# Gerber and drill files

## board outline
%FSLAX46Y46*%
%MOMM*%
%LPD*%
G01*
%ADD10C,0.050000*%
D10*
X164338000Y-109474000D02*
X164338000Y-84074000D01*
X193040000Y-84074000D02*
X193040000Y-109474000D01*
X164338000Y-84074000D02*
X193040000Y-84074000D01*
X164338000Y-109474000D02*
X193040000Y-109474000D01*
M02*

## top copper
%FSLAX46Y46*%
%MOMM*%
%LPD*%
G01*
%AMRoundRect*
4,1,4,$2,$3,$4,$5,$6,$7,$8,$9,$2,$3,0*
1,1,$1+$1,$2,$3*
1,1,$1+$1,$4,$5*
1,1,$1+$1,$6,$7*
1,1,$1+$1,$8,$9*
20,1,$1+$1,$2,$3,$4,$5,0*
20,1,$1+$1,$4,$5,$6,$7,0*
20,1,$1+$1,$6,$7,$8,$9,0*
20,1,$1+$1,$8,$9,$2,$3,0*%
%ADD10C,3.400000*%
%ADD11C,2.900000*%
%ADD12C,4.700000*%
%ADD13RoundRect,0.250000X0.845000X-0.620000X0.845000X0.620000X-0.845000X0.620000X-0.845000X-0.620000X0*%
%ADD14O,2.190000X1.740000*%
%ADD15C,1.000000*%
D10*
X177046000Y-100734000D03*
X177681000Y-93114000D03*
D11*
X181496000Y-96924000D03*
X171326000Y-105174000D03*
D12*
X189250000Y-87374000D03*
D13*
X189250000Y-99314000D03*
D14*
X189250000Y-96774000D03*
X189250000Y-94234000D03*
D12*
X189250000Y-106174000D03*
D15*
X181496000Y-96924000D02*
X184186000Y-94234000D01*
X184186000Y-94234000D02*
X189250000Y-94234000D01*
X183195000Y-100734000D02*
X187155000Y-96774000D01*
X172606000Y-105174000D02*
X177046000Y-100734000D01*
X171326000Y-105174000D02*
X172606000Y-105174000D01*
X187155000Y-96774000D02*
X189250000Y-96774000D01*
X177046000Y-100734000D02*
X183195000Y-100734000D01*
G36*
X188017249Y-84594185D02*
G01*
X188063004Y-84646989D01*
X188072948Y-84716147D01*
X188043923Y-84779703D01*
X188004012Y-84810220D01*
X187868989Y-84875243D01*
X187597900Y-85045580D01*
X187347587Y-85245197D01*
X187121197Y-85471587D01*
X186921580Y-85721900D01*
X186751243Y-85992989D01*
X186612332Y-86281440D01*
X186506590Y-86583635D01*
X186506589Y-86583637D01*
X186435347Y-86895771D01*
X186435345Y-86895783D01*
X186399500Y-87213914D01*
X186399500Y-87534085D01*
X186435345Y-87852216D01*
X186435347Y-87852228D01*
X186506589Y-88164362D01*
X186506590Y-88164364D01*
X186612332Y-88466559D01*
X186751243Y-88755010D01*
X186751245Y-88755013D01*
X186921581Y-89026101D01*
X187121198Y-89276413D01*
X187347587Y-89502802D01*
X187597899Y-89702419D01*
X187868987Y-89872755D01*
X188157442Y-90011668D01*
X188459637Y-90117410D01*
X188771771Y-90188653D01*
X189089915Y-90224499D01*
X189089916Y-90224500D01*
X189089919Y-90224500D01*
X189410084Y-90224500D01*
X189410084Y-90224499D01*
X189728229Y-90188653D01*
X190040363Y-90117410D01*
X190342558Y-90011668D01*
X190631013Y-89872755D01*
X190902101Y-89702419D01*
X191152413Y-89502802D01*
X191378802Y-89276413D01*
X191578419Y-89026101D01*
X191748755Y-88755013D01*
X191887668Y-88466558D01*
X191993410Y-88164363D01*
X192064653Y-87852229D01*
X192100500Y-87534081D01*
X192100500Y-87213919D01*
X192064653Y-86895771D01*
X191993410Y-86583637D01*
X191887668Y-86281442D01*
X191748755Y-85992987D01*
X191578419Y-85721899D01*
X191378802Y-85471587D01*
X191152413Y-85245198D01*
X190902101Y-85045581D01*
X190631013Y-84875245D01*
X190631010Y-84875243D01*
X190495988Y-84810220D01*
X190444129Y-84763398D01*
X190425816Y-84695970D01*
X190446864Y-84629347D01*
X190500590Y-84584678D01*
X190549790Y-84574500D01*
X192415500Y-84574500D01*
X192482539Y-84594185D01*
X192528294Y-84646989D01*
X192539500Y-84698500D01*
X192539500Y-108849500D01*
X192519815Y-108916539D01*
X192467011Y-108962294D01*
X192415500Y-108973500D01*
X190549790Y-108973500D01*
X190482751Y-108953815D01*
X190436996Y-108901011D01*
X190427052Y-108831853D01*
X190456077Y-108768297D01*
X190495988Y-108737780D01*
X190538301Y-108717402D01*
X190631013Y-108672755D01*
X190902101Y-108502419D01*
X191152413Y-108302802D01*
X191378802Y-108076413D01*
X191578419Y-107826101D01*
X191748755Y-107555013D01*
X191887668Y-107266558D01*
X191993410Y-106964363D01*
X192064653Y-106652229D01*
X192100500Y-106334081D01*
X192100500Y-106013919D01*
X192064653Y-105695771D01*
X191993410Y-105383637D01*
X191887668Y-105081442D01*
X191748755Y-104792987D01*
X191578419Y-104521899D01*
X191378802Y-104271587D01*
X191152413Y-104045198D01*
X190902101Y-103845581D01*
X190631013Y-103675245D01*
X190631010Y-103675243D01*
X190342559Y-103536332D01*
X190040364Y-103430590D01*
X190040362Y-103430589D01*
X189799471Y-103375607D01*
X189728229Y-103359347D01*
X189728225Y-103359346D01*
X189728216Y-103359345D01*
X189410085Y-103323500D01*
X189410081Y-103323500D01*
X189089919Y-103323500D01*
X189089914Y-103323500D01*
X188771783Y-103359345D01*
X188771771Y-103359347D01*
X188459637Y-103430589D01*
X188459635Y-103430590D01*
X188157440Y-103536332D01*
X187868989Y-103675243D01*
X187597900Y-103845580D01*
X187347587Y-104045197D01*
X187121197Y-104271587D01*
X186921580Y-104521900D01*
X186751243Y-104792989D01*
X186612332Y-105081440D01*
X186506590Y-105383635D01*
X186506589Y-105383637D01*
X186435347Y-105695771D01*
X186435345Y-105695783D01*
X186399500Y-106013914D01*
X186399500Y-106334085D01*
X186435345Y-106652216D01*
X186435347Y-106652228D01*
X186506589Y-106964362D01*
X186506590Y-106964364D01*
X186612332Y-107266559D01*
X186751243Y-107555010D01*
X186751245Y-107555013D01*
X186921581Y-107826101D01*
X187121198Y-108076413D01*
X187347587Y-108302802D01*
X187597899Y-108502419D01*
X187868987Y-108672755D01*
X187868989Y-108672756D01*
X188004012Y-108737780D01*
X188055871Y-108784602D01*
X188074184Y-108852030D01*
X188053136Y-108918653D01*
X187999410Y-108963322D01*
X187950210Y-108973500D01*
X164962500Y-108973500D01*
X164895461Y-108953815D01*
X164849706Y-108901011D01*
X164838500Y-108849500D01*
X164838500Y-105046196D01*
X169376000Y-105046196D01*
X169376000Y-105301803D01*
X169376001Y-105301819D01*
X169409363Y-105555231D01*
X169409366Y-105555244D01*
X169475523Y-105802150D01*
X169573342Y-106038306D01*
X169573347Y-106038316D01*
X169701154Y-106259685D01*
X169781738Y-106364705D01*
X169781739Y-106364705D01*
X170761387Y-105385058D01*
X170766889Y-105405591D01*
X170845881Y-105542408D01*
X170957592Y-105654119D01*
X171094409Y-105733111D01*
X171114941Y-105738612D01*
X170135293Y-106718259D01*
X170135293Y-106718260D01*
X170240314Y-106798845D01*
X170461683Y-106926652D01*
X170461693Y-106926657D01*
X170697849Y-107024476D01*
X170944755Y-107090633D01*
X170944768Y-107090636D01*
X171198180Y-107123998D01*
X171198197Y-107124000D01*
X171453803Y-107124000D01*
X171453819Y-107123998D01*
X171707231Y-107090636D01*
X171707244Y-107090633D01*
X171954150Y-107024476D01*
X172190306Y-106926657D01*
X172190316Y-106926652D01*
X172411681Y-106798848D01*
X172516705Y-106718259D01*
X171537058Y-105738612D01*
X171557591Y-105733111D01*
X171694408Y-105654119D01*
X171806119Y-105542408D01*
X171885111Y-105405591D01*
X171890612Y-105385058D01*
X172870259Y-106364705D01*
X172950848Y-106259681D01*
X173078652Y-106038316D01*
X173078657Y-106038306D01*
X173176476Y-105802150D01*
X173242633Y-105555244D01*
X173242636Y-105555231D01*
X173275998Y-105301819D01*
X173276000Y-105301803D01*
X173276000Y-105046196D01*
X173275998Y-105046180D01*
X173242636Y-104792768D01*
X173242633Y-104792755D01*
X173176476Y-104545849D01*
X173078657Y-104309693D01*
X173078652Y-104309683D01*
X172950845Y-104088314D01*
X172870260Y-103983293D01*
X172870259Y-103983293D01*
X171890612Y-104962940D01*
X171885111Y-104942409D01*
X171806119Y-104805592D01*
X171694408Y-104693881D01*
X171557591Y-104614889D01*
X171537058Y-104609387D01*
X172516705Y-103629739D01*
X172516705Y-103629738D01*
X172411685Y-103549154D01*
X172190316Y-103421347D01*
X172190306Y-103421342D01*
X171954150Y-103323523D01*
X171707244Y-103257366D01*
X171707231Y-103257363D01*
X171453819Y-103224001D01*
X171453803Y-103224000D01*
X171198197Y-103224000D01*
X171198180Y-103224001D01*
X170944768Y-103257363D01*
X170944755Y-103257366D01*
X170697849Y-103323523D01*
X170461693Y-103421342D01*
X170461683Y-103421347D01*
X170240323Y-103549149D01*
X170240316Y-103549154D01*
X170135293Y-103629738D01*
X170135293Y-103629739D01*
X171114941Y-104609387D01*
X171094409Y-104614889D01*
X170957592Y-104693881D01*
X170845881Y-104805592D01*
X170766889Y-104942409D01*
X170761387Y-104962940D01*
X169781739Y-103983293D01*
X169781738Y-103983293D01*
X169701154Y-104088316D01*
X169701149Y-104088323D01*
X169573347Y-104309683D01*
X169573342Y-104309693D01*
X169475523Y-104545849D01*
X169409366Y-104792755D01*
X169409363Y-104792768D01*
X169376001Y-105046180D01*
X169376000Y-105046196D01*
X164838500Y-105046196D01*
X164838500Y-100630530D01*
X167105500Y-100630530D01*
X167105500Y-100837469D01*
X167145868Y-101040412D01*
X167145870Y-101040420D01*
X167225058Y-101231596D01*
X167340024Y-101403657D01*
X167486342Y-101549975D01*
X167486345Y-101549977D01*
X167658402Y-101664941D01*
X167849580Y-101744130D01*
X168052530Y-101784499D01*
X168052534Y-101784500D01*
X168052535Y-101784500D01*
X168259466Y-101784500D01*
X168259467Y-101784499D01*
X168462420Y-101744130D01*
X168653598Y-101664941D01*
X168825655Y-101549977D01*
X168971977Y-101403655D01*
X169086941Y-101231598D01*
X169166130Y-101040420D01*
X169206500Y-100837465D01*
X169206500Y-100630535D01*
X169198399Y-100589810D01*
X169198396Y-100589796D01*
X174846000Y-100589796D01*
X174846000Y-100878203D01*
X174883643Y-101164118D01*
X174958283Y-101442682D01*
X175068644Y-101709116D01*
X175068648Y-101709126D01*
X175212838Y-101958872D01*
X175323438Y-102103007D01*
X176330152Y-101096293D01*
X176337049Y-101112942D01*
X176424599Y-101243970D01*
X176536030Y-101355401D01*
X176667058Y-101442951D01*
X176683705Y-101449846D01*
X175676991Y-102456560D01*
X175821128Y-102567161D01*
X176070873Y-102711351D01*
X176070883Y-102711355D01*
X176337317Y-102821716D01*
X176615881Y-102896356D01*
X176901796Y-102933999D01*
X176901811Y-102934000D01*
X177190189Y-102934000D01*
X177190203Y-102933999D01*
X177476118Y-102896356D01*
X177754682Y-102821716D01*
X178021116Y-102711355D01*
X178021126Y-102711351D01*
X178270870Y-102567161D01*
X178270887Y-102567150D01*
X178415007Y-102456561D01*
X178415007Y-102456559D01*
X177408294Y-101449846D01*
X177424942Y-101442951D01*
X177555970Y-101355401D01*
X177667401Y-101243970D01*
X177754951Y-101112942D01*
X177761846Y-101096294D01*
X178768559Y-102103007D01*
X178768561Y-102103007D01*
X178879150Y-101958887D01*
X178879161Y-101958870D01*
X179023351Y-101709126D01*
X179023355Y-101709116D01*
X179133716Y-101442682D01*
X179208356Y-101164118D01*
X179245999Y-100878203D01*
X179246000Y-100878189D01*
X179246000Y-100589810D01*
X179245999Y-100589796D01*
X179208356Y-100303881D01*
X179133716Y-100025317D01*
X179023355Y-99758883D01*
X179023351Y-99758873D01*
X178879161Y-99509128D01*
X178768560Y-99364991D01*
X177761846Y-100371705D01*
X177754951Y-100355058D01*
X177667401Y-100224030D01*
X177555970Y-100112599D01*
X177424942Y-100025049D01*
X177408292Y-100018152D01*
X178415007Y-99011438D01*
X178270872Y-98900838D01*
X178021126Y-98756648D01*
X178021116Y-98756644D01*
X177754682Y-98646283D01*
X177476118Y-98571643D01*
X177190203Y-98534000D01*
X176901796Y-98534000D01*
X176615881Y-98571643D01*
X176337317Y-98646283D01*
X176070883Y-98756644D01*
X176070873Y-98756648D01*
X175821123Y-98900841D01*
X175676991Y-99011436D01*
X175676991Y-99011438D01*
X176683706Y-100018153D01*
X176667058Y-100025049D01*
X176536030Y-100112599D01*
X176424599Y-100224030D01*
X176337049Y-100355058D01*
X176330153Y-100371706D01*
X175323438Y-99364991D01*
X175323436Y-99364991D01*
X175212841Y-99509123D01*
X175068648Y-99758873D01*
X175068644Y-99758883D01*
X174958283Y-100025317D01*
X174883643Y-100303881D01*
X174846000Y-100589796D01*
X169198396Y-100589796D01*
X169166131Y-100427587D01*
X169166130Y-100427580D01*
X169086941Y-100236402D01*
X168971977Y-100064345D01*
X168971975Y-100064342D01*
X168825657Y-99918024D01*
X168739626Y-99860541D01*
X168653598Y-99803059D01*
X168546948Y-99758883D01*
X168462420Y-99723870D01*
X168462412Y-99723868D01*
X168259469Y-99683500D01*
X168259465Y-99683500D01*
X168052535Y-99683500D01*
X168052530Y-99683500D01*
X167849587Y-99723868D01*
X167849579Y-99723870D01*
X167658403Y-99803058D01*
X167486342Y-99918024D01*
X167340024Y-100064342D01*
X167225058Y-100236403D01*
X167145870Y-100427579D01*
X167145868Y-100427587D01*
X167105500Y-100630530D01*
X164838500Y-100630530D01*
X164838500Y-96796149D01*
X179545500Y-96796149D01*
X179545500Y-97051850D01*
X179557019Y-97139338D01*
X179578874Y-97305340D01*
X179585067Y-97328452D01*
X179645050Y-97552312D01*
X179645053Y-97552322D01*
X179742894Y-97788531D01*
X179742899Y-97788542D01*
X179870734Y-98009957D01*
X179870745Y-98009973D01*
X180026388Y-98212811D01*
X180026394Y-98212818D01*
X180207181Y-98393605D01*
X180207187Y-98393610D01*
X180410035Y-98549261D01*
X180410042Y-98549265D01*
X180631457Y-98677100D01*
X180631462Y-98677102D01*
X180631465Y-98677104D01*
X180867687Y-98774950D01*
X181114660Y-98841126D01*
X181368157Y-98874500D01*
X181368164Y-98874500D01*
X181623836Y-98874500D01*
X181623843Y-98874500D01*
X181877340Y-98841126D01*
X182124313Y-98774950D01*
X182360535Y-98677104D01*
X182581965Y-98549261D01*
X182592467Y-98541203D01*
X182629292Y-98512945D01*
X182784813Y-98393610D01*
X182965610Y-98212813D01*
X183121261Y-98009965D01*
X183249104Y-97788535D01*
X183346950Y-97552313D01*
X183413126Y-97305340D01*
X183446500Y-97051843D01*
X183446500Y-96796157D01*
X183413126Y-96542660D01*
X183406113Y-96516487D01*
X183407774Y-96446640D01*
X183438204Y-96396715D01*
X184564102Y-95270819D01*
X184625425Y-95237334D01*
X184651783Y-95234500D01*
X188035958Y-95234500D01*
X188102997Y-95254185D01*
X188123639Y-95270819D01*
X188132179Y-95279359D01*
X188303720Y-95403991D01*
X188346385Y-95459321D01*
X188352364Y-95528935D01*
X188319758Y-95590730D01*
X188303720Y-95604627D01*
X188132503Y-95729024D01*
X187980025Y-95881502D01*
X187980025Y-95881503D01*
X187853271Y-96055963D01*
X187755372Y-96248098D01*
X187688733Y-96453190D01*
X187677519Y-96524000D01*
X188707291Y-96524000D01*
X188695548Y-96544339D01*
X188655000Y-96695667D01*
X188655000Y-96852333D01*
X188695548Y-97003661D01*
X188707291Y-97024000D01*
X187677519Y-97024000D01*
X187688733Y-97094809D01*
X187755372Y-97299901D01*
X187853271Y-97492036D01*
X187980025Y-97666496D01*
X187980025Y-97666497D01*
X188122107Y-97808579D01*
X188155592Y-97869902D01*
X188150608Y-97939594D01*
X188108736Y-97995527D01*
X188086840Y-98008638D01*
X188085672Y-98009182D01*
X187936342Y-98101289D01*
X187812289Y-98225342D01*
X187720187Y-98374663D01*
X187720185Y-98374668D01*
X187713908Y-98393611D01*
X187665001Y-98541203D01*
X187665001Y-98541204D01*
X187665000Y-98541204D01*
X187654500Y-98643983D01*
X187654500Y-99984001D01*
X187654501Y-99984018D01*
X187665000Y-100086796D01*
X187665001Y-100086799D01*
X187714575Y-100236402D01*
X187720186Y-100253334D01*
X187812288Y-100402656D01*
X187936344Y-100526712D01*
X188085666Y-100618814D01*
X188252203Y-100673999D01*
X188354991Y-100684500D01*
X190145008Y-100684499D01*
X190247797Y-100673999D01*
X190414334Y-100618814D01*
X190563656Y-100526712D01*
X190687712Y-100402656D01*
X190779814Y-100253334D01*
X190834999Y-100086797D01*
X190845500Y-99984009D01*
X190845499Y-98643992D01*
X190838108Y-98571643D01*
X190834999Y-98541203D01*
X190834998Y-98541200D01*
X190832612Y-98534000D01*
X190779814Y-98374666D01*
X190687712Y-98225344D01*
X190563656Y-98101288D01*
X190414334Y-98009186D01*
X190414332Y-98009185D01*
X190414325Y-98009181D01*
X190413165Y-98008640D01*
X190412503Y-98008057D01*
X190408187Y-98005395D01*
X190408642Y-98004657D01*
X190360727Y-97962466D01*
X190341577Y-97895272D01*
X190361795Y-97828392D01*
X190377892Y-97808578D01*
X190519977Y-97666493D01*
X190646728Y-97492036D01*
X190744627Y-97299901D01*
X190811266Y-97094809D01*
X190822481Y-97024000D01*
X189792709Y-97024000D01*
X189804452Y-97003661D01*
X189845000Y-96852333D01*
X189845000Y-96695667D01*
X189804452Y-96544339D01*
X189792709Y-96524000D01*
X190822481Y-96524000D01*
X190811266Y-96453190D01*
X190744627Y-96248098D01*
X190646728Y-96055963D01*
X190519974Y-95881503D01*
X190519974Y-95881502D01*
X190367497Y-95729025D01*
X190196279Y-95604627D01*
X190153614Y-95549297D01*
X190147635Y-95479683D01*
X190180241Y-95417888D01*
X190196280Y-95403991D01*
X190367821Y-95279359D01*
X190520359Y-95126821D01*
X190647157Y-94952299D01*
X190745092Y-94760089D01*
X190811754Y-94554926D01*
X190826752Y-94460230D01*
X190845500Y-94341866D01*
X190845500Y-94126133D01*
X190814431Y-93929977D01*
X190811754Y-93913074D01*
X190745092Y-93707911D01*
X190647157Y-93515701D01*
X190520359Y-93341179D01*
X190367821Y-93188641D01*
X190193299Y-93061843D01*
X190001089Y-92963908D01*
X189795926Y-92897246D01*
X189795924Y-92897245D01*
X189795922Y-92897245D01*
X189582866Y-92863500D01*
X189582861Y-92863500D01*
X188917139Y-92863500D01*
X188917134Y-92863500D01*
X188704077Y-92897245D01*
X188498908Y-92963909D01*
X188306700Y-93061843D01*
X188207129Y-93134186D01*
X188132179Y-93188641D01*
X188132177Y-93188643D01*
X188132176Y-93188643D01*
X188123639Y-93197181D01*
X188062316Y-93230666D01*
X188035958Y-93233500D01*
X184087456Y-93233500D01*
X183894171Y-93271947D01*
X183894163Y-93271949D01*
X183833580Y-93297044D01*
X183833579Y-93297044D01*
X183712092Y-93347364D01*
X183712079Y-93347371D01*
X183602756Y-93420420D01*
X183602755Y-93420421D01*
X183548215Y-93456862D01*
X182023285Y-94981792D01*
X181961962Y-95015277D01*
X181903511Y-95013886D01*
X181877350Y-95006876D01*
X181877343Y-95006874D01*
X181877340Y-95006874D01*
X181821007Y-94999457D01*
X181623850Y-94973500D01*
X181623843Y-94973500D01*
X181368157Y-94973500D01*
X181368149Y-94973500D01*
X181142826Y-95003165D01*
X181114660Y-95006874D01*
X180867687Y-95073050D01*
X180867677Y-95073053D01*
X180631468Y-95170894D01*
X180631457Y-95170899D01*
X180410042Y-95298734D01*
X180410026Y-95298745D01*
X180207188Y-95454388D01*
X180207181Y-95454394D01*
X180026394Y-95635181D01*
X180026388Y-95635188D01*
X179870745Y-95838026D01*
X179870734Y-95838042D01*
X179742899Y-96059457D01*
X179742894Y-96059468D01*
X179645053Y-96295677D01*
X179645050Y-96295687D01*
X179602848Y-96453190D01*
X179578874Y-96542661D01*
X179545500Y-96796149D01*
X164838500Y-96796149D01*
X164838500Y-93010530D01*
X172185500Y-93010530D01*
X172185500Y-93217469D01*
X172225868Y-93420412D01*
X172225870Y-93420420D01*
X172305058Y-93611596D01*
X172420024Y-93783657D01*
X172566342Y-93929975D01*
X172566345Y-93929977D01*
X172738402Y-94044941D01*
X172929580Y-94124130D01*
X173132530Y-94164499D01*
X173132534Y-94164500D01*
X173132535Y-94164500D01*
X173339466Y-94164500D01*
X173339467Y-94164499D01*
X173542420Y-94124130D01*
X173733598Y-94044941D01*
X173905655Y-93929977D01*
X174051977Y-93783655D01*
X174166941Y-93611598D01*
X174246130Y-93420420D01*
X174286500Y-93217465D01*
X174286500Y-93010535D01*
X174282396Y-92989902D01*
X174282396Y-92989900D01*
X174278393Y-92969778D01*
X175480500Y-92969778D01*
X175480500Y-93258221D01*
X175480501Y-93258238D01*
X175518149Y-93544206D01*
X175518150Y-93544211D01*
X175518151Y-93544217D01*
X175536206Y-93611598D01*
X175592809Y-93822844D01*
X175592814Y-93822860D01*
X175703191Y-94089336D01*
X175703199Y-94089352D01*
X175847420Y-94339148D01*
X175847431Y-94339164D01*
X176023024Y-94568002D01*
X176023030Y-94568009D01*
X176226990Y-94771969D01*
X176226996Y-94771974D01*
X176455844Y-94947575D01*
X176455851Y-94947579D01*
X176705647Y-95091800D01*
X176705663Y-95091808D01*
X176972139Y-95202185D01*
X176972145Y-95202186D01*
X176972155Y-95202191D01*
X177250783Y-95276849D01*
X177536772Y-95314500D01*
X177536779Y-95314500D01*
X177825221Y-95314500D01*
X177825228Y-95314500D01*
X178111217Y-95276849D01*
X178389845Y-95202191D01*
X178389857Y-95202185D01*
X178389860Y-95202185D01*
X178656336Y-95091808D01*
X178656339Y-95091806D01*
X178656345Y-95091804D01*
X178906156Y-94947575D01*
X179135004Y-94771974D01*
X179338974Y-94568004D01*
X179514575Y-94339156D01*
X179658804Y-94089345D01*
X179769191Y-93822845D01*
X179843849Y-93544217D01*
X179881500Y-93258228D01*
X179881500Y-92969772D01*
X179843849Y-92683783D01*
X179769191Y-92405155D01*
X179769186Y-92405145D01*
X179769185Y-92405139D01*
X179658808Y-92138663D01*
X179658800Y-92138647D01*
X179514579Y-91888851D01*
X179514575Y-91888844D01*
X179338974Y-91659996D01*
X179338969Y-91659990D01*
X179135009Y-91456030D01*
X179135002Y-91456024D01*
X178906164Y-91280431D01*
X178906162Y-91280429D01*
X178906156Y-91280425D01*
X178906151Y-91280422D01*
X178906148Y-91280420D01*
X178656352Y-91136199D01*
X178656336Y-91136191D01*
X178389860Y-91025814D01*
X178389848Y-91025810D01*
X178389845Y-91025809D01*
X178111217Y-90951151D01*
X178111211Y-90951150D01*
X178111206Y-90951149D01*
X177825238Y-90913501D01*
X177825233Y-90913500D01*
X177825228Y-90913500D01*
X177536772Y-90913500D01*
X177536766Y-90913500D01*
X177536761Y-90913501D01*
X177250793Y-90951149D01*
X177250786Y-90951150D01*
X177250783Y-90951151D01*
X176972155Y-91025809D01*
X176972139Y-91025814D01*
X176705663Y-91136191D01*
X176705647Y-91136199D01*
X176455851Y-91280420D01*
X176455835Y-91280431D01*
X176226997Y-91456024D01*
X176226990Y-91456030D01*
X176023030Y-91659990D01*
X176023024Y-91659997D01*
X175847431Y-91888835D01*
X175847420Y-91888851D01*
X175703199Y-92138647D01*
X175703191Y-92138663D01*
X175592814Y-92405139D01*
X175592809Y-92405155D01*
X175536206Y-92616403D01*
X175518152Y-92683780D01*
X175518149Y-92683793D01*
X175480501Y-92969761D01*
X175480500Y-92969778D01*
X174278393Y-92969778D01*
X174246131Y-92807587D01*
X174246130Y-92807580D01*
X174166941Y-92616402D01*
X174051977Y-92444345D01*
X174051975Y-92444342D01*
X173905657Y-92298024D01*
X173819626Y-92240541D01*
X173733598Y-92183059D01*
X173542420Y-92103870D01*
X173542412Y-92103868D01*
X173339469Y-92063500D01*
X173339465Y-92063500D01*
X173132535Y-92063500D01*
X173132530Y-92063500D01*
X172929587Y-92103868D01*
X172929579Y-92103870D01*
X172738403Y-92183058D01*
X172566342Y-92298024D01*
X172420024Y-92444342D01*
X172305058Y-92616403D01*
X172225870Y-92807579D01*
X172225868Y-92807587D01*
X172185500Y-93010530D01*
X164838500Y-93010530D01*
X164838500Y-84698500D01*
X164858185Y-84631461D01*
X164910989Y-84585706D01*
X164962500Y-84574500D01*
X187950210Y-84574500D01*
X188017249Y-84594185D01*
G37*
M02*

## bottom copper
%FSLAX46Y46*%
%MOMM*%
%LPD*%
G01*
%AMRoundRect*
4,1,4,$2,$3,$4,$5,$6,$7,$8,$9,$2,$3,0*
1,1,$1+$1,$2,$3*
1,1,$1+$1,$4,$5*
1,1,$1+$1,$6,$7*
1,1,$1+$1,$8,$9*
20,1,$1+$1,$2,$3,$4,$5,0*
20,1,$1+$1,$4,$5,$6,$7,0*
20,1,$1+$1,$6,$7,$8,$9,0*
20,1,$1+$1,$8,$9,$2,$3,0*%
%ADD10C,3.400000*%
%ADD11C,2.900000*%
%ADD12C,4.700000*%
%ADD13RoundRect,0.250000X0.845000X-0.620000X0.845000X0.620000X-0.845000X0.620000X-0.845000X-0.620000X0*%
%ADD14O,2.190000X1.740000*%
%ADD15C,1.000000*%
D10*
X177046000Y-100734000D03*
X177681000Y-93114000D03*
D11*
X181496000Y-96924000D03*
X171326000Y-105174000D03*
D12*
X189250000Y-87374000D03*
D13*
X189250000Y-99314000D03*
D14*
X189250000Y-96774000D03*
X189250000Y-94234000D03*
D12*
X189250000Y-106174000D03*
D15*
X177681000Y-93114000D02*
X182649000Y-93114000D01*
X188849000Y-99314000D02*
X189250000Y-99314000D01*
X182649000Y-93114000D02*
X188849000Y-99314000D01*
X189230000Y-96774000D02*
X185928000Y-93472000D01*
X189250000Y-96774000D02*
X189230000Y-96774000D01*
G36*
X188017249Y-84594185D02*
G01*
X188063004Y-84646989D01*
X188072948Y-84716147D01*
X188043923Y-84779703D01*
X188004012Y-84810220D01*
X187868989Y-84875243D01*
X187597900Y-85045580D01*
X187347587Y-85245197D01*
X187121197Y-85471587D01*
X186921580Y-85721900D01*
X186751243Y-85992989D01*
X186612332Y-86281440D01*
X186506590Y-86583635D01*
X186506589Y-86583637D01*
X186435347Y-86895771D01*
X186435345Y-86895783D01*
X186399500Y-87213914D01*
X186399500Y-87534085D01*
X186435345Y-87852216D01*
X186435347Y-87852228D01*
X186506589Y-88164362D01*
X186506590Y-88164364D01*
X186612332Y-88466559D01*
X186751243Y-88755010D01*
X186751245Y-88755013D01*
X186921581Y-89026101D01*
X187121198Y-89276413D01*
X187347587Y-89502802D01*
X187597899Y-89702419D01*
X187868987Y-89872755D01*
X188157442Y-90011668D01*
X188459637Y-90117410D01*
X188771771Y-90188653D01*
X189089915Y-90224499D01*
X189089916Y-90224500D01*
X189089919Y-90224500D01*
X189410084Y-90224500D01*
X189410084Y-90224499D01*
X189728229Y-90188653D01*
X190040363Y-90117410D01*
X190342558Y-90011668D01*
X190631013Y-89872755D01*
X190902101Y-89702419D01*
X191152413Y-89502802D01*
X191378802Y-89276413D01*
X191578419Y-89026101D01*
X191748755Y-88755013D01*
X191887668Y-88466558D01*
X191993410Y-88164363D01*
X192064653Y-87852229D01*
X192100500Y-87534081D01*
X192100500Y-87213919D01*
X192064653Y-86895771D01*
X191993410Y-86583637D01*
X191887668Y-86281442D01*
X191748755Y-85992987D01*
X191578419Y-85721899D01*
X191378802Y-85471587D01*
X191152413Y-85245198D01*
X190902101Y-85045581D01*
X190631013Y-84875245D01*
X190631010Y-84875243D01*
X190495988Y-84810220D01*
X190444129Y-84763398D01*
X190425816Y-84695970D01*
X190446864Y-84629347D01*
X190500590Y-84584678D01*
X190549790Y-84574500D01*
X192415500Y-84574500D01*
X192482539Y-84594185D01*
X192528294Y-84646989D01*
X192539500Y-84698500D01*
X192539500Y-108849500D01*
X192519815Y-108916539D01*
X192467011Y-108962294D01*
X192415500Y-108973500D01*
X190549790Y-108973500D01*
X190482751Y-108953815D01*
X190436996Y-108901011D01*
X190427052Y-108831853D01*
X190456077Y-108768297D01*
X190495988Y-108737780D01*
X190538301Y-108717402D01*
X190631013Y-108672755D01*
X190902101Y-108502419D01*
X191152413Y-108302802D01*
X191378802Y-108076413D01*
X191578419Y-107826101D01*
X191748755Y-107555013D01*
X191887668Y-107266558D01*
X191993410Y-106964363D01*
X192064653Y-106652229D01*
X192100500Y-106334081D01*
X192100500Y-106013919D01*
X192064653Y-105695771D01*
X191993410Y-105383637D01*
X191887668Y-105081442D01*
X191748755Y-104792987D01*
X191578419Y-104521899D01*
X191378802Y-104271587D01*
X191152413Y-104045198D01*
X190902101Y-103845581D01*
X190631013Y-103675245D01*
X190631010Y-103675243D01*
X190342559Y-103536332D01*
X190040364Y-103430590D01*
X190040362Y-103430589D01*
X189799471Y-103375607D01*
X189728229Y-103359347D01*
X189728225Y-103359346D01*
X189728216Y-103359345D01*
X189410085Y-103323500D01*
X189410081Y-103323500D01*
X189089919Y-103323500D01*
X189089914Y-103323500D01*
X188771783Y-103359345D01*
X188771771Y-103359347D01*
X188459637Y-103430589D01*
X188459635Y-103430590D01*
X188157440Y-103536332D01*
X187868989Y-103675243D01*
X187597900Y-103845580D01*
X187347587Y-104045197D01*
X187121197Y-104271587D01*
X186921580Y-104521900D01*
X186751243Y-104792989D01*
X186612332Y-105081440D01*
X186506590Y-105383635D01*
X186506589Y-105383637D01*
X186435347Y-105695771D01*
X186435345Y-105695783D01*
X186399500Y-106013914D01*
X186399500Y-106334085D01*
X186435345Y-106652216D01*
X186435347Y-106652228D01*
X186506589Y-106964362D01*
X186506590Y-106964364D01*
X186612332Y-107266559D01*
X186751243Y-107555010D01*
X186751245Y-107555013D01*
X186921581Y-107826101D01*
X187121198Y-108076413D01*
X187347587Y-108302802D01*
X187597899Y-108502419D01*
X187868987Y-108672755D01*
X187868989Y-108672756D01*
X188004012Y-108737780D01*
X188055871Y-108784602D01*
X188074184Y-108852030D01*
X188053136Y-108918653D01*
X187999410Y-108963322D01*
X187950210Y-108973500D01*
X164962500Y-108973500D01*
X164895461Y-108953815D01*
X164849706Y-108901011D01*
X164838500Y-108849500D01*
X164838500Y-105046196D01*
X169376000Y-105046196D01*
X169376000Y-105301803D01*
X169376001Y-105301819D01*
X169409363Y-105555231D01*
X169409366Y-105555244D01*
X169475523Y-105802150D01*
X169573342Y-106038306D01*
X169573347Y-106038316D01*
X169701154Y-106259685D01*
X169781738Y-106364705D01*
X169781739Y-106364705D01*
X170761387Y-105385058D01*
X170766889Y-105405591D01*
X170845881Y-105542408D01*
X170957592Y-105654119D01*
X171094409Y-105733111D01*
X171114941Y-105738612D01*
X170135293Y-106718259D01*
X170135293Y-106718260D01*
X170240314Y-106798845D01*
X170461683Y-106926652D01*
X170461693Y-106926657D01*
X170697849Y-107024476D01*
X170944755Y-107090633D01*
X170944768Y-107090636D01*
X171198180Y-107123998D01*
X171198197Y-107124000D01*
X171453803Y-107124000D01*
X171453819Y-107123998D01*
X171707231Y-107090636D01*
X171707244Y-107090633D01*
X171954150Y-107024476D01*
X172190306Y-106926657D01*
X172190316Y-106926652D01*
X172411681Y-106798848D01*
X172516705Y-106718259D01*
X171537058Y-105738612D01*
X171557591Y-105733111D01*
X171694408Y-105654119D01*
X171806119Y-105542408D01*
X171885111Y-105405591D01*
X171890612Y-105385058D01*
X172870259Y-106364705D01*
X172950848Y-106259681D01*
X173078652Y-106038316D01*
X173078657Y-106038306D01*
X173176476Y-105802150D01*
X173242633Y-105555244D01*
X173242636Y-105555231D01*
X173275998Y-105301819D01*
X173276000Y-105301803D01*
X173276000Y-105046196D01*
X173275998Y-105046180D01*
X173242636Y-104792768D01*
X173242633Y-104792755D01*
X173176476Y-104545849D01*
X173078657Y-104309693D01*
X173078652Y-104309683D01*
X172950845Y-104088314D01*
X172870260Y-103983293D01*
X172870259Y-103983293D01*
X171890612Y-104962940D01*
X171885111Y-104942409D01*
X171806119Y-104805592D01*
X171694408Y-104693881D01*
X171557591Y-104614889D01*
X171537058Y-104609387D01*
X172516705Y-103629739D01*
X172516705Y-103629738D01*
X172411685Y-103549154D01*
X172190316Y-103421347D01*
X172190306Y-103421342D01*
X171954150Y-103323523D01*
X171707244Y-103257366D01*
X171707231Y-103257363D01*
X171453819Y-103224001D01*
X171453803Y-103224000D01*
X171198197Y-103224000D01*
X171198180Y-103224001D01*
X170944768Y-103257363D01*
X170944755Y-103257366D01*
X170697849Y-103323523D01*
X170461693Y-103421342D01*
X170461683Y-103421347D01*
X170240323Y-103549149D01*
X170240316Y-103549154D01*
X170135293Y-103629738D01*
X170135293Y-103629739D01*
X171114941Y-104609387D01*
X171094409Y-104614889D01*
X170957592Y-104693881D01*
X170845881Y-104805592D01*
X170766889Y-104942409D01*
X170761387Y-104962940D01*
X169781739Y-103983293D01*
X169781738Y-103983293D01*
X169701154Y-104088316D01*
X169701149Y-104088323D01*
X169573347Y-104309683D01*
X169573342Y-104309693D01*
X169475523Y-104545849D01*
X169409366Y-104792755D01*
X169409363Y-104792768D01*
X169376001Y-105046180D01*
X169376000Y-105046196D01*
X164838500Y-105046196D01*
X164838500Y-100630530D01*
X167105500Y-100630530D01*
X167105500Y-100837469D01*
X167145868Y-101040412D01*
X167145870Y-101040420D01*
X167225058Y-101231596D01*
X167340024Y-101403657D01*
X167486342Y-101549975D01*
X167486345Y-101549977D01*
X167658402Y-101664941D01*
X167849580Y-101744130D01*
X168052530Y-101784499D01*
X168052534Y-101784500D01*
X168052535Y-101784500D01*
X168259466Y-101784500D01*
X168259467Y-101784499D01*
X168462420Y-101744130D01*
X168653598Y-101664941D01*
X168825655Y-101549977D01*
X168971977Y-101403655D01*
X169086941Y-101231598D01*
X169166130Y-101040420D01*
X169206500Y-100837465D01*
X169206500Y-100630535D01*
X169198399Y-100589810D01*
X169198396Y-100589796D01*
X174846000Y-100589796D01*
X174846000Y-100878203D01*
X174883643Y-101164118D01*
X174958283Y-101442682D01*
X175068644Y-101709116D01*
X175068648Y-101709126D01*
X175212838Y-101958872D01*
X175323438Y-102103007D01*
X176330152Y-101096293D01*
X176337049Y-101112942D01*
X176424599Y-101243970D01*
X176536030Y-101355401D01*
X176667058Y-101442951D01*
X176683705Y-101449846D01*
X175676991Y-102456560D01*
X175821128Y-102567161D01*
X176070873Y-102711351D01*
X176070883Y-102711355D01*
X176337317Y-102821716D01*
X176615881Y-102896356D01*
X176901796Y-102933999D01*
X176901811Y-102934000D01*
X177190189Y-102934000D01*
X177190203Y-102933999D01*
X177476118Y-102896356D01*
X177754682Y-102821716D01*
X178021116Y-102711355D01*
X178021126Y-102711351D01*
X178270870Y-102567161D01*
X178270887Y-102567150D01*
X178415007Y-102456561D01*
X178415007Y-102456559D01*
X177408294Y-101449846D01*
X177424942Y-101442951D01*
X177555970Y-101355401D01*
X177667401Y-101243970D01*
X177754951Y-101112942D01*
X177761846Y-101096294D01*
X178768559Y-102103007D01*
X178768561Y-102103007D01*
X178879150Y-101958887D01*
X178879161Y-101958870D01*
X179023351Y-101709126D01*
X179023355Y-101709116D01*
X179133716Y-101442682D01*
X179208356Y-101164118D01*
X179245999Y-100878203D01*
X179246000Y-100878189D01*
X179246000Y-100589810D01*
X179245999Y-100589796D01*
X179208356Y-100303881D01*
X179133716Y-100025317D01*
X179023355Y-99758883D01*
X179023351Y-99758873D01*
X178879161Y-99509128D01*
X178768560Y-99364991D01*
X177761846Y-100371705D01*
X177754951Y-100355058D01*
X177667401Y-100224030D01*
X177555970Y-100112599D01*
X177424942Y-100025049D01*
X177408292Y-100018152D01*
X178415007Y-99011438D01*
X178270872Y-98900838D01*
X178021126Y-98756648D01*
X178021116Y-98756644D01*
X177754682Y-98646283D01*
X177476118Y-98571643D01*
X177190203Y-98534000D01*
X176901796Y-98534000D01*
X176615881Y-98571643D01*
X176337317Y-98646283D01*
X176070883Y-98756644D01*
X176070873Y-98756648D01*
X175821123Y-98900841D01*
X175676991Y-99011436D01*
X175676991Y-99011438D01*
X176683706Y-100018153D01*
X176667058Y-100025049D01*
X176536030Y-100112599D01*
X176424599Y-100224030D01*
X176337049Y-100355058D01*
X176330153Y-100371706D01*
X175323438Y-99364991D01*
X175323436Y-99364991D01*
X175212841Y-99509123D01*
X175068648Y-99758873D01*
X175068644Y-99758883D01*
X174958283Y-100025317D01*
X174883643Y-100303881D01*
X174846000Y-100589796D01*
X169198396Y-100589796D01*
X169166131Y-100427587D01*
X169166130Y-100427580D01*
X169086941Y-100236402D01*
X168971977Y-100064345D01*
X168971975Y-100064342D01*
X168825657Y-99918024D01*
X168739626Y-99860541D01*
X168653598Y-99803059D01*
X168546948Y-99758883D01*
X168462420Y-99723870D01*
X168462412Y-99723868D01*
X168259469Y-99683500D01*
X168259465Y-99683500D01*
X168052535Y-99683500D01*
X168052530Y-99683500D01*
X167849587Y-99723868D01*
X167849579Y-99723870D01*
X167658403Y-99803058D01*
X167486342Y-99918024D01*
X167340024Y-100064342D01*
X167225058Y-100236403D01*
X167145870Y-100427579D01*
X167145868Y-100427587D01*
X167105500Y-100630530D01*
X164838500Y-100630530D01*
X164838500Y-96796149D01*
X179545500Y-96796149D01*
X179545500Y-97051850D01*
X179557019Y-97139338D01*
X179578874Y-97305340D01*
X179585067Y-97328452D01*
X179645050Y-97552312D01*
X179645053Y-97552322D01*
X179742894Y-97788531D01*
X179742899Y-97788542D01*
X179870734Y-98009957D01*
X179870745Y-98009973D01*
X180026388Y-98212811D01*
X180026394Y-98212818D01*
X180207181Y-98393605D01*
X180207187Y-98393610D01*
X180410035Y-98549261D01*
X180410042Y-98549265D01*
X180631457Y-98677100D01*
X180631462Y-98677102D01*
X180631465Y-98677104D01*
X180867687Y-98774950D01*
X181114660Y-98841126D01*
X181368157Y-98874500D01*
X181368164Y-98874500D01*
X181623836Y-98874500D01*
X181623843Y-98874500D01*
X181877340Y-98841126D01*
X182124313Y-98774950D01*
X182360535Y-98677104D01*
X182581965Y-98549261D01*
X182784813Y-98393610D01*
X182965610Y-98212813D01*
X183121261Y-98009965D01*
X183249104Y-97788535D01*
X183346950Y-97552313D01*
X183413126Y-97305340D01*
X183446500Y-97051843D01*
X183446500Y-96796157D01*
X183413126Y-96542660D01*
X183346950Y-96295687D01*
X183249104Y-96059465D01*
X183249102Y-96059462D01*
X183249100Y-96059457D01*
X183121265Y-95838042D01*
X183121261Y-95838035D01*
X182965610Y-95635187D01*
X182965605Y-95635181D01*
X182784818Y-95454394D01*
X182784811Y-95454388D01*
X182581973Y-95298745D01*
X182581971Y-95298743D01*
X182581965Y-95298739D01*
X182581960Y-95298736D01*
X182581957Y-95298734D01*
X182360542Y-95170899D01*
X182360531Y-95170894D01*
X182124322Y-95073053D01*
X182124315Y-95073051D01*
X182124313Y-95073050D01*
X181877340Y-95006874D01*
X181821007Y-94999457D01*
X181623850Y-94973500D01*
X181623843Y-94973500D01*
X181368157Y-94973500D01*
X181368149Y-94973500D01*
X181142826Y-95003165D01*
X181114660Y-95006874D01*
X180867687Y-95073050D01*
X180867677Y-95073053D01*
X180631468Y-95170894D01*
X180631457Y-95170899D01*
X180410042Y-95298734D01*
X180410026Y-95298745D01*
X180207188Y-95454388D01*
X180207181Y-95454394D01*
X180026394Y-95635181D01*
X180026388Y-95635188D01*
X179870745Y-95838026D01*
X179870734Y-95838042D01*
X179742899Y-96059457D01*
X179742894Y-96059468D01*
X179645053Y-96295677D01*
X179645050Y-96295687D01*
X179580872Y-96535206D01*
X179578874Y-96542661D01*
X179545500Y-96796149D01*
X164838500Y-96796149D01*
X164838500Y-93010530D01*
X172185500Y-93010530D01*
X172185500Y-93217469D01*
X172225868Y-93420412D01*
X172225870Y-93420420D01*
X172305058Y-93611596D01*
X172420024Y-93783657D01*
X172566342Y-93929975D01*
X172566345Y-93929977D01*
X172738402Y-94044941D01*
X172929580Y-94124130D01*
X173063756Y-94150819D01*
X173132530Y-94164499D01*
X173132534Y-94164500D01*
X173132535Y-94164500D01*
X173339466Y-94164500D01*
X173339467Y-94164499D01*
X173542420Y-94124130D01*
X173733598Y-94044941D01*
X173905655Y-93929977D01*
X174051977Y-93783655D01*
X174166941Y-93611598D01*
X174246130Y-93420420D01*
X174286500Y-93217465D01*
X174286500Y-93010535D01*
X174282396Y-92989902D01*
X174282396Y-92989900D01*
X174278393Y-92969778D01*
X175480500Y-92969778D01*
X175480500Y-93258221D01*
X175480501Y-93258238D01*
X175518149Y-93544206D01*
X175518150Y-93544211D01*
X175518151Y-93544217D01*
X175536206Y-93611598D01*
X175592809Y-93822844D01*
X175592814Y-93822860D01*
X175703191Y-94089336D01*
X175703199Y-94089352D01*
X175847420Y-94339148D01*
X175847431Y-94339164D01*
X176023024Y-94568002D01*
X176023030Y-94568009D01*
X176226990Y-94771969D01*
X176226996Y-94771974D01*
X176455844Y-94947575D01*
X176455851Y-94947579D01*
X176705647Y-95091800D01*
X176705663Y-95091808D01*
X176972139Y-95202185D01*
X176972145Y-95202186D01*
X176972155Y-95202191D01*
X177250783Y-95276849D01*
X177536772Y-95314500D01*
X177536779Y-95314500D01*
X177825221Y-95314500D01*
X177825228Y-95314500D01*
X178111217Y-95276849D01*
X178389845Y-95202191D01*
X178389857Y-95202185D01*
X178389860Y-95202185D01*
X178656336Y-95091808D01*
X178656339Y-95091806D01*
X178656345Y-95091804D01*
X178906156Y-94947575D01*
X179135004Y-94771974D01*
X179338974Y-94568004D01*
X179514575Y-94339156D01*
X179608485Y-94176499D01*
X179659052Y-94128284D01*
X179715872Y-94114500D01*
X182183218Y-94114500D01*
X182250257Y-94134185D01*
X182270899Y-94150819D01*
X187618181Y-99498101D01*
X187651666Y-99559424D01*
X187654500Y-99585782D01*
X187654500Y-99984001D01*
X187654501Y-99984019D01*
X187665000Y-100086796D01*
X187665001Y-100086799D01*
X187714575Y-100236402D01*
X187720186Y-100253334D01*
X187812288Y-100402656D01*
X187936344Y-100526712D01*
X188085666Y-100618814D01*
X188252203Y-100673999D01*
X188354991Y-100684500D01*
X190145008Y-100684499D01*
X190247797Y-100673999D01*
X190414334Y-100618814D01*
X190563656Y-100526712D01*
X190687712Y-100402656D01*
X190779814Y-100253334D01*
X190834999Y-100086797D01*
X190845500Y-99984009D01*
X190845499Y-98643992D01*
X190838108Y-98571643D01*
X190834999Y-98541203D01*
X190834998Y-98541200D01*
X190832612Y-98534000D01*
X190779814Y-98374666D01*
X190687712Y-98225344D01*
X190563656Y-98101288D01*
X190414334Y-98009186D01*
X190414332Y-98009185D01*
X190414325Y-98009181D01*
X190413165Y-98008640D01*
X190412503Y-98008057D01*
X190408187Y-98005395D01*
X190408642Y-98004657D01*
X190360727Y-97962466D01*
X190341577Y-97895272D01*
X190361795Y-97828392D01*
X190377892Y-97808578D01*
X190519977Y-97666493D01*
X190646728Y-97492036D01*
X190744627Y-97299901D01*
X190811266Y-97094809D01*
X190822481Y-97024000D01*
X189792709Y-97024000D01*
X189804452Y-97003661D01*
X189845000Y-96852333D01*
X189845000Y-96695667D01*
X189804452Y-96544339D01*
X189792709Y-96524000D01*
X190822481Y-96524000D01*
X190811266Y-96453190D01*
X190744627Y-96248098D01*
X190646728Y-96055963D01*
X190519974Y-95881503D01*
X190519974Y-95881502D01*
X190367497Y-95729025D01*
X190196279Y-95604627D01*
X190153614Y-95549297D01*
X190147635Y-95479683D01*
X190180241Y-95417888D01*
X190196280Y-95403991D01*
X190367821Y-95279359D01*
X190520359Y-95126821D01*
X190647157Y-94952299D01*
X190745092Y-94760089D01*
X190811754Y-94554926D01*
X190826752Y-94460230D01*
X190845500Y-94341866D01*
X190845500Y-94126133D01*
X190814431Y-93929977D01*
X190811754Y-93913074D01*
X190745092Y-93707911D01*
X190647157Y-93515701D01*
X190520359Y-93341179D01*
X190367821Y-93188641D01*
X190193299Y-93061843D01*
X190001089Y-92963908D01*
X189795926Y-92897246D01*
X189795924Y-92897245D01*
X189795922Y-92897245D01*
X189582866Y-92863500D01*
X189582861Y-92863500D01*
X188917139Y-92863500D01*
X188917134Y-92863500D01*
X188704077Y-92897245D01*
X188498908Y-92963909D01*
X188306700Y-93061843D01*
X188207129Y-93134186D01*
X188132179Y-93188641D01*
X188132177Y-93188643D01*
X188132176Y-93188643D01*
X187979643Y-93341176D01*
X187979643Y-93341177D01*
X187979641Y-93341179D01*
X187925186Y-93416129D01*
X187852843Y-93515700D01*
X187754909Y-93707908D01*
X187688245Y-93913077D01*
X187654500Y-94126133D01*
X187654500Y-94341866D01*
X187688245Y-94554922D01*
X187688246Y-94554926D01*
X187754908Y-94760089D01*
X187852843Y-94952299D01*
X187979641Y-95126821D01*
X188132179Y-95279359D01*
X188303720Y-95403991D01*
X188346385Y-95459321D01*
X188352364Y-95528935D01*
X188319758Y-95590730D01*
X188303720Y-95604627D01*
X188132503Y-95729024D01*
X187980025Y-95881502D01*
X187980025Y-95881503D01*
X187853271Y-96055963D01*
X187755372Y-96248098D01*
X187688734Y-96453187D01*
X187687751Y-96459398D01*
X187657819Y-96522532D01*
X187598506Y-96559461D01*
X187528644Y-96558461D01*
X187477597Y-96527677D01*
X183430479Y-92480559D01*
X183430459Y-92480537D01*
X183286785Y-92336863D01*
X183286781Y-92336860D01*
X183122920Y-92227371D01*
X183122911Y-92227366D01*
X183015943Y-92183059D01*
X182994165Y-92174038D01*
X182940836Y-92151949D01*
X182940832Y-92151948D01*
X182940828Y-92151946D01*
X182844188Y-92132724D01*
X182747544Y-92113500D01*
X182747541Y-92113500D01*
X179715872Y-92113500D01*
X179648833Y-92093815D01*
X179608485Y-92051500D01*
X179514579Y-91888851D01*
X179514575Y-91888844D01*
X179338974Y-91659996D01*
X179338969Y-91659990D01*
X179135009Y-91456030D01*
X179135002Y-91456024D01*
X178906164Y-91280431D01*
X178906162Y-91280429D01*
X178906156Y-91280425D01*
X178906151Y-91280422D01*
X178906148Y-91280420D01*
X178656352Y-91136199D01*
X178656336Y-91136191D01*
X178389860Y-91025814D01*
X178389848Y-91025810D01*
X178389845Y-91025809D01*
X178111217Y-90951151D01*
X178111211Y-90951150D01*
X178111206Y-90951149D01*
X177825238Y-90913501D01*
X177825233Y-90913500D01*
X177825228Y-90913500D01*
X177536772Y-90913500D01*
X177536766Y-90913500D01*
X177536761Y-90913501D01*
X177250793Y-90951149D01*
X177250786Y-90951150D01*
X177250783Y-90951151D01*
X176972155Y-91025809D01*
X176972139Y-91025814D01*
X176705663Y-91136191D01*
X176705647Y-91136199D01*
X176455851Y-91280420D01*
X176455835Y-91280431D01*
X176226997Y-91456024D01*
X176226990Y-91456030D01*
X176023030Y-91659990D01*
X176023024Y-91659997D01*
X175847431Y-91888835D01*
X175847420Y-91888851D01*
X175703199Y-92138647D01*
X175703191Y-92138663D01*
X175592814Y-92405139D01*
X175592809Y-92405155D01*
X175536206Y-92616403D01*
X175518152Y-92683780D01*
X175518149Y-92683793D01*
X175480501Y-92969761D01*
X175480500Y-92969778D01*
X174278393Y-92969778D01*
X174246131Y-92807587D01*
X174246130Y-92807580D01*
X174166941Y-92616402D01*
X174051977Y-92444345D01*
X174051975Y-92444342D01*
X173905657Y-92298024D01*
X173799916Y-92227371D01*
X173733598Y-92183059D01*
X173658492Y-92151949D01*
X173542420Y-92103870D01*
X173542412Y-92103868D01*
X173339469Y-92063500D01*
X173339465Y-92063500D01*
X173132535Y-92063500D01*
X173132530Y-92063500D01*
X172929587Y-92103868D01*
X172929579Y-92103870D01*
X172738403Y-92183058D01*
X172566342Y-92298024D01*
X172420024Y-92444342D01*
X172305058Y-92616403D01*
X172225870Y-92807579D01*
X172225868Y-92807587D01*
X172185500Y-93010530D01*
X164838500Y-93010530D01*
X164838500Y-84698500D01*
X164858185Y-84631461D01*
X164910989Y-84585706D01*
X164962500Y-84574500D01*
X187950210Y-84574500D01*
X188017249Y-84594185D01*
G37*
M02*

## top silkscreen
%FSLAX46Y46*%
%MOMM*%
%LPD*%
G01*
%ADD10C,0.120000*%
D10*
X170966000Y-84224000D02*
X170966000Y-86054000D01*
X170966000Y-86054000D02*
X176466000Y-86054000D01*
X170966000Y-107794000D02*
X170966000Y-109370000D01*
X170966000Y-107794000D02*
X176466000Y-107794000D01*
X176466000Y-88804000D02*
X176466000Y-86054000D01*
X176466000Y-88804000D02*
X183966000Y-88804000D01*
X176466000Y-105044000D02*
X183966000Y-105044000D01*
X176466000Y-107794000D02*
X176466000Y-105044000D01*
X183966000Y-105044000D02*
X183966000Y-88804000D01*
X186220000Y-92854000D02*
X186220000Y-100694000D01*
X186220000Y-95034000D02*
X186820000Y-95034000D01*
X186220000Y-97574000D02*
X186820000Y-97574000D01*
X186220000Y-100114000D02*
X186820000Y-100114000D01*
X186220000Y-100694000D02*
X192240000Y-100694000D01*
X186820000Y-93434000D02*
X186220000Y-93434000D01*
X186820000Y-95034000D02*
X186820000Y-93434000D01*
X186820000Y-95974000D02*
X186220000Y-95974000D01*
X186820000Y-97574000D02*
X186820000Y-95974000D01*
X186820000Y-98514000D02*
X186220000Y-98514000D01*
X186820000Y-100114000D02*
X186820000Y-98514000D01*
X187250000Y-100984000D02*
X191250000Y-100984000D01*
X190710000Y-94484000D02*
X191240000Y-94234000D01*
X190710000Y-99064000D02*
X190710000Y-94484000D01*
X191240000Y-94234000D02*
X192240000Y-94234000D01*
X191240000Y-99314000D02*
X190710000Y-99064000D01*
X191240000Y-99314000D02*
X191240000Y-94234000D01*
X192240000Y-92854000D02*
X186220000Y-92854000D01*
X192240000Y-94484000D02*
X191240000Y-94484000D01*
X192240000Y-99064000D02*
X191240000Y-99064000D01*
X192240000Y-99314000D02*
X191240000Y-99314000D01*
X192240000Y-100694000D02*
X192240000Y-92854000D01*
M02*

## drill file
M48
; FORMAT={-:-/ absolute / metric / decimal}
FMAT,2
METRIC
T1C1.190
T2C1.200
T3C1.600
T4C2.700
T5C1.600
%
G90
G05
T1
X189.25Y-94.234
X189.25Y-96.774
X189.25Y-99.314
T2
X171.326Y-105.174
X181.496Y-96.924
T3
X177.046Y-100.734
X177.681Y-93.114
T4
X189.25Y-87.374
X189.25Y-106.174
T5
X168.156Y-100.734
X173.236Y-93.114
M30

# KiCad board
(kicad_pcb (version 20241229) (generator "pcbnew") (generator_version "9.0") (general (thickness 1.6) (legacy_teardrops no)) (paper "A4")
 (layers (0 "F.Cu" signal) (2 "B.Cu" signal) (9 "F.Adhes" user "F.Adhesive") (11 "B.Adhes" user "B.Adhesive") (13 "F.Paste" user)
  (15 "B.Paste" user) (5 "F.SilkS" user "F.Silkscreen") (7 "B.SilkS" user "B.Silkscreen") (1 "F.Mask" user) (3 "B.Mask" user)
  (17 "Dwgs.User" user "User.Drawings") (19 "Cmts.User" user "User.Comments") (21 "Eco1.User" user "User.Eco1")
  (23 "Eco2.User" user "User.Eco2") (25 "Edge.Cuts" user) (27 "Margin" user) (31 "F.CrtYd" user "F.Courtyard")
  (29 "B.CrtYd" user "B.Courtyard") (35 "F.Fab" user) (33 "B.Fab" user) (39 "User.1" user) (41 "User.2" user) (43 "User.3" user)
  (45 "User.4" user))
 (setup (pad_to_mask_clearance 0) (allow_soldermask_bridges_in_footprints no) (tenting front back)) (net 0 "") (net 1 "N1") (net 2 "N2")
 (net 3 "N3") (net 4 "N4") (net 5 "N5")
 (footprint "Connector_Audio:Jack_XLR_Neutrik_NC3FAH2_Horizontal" (layer "F.Cu") (at 177.046 100.734 180)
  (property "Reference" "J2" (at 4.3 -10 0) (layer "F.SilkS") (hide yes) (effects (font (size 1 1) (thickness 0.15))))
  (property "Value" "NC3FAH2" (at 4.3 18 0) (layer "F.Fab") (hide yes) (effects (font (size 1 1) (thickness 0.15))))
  (fp_line (start 6.08 16.51) (end 6.08 14.68) (stroke (width 0.12) (type solid)) (layer "F.SilkS"))
  (fp_line (start 6.08 14.68) (end 0.58 14.68) (stroke (width 0.12) (type solid)) (layer "F.SilkS"))
  (fp_line (start 6.08 -7.06) (end 6.08 -8.636) (stroke (width 0.12) (type solid)) (layer "F.SilkS"))
  (fp_line (start 6.08 -7.06) (end 0.58 -7.06) (stroke (width 0.12) (type solid)) (layer "F.SilkS"))
  (fp_line (start 0.58 11.93) (end 0.58 14.68) (stroke (width 0.12) (type solid)) (layer "F.SilkS"))
  (fp_line (start 0.58 11.93) (end -6.92 11.93) (stroke (width 0.12) (type solid)) (layer "F.SilkS"))
  (fp_line (start 0.58 -4.31) (end -6.92 -4.31) (stroke (width 0.12) (type solid)) (layer "F.SilkS"))
  (fp_line (start 0.58 -7.06) (end 0.58 -4.31) (stroke (width 0.12) (type solid)) (layer "F.SilkS"))
  (fp_line (start -6.92 -4.31) (end -6.92 11.93) (stroke (width 0.12) (type solid)) (layer "F.SilkS"))
  (pad "" np_thru_hole circle (at 3.81 7.62 180) (size 1.6 1.6) (drill 1.6) (layers "*.Cu" "*.Mask"))
  (pad "" np_thru_hole circle (at 8.89 0 180) (size 1.6 1.6) (drill 1.6) (layers "*.Cu" "*.Mask"))
  (pad "1" thru_hole circle (at 0 0 180) (size 3.4 3.4) (drill 1.6) (layers "*.Cu" "*.Mask") (remove_unused_layers no) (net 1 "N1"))
  (pad "2" thru_hole circle (at -0.635 7.62 180) (size 3.4 3.4) (drill 1.6) (layers "*.Cu" "*.Mask") (remove_unused_layers no) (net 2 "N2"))
  (pad "3" thru_hole circle (at -4.45 3.81 180) (size 2.9 2.9) (drill 1.2) (layers "*.Cu" "*.Mask") (remove_unused_layers no) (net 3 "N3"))
  (pad "G" thru_hole circle (at 5.72 -4.44 180) (size 2.9 2.9) (drill 1.2) (layers "*.Cu" "*.Mask") (remove_unused_layers no) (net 1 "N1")))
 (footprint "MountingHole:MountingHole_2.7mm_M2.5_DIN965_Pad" (layer "F.Cu") (at 189.25 87.374)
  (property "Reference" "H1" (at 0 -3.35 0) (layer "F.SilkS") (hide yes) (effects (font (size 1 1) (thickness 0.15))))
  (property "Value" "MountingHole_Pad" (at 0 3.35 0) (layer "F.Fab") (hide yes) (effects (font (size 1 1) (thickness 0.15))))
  (pad "1" thru_hole circle (at 0 0) (size 4.7 4.7) (drill 2.7) (layers "*.Cu" "*.Mask") (remove_unused_layers no) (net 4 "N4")))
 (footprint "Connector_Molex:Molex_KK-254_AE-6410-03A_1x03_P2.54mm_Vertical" (layer "F.Cu") (at 189.25 99.314 90)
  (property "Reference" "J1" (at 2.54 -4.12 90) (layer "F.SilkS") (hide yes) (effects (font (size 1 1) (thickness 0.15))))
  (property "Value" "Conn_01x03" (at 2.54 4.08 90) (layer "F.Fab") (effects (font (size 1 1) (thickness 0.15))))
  (fp_line (start 6.46 -3.03) (end -1.38 -3.03) (stroke (width 0.12) (type solid)) (layer "F.SilkS"))
  (fp_line (start 4.28 -3.03) (end 4.28 -2.43) (stroke (width 0.12) (type solid)) (layer "F.SilkS"))
  (fp_line (start 1.74 -3.03) (end 1.74 -2.43) (stroke (width 0.12) (type solid)) (layer "F.SilkS"))
  (fp_line (start -0.8 -3.03) (end -0.8 -2.43) (stroke (width 0.12) (type solid)) (layer "F.SilkS"))
  (fp_line (start -1.38 -3.03) (end -1.38 2.99) (stroke (width 0.12) (type solid)) (layer "F.SilkS"))
  (fp_line (start 5.88 -2.43) (end 5.88 -3.03) (stroke (width 0.12) (type solid)) (layer "F.SilkS"))
  (fp_line (start 4.28 -2.43) (end 5.88 -2.43) (stroke (width 0.12) (type solid)) (layer "F.SilkS"))
  (fp_line (start 3.34 -2.43) (end 3.34 -3.03) (stroke (width 0.12) (type solid)) (layer "F.SilkS"))
  (fp_line (start 1.74 -2.43) (end 3.34 -2.43) (stroke (width 0.12) (type solid)) (layer "F.SilkS"))
  (fp_line (start 0.8 -2.43) (end 0.8 -3.03) (stroke (width 0.12) (type solid)) (layer "F.SilkS"))
  (fp_line (start -0.8 -2.43) (end 0.8 -2.43) (stroke (width 0.12) (type solid)) (layer "F.SilkS"))
  (fp_line (start -1.67 -2) (end -1.67 2) (stroke (width 0.12) (type solid)) (layer "F.SilkS"))
  (fp_line (start 4.83 1.46) (end 5.08 1.99) (stroke (width 0.12) (type solid)) (layer "F.SilkS"))
  (fp_line (start 0.25 1.46) (end 4.83 1.46) (stroke (width 0.12) (type solid)) (layer "F.SilkS"))
  (fp_line (start 5.08 1.99) (end 5.08 2.99) (stroke (width 0.12) (type solid)) (layer "F.SilkS"))
  (fp_line (start 0 1.99) (end 0.25 1.46) (stroke (width 0.12) (type solid)) (layer "F.SilkS"))
  (fp_line (start 0 1.99) (end 5.08 1.99) (stroke (width 0.12) (type solid)) (layer "F.SilkS"))
  (fp_line (start 6.46 2.99) (end 6.46 -3.03) (stroke (width 0.12) (type solid)) (layer "F.SilkS"))
  (fp_line (start 4.83 2.99) (end 4.83 1.99) (stroke (width 0.12) (type solid)) (layer "F.SilkS"))
  (fp_line (start 0.25 2.99) (end 0.25 1.99) (stroke (width 0.12) (type solid)) (layer "F.SilkS"))
  (fp_line (start 0 2.99) (end 0 1.99) (stroke (width 0.12) (type solid)) (layer "F.SilkS"))
  (fp_line (start -1.38 2.99) (end 6.46 2.99) (stroke (width 0.12) (type solid)) (layer "F.SilkS"))
  (pad "1" thru_hole roundrect (at 0 0 90) (size 1.74 2.19) (drill 1.19) (layers "*.Cu" "*.Mask") (remove_unused_layers no)
   (roundrect_rratio 0.143678) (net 2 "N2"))
  (pad "2" thru_hole oval (at 2.54 0 90) (size 1.74 2.19) (drill 1.19) (layers "*.Cu" "*.Mask") (remove_unused_layers no) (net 1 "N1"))
  (pad "3" thru_hole oval (at 5.08 0 90) (size 1.74 2.19) (drill 1.19) (layers "*.Cu" "*.Mask") (remove_unused_layers no) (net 3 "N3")))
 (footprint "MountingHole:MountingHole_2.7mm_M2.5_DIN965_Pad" (layer "F.Cu") (at 189.23 106.174)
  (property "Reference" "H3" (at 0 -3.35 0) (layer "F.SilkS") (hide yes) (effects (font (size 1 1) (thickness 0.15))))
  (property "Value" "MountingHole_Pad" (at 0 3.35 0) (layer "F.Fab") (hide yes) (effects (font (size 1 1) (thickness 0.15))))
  (pad "1" thru_hole circle (at 0.02 0) (size 4.7 4.7) (drill 2.7) (layers "*.Cu" "*.Mask") (remove_unused_layers no) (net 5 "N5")))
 (gr_line (start 164.338 109.474) (end 164.338 84.074) (stroke (width 0.05) (type default)) (layer "Edge.Cuts"))
 (gr_line (start 193.04 84.074) (end 193.04 109.474) (stroke (width 0.05) (type default)) (layer "Edge.Cuts"))
 (gr_line (start 164.338 84.074) (end 193.04 84.074) (stroke (width 0.05) (type default)) (layer "Edge.Cuts"))
 (gr_line (start 164.338 109.474) (end 193.04 109.474) (stroke (width 0.05) (type default)) (layer "Edge.Cuts"))
 (segment (start 181.496 96.924) (end 184.186 94.234) (width 1) (layer "F.Cu") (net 3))
 (segment (start 184.186 94.234) (end 189.25 94.234) (width 1) (layer "F.Cu") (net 3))
 (segment (start 177.681 93.114) (end 182.649 93.114) (width 1) (layer "B.Cu") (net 2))
 (segment (start 188.849 99.314) (end 189.25 99.314) (width 1) (layer "B.Cu") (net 2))
 (segment (start 182.649 93.114) (end 188.849 99.314) (width 1) (layer "B.Cu") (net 2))
 (segment (start 183.195 100.734) (end 187.155 96.774) (width 1) (layer "F.Cu") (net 1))
 (segment (start 172.606 105.174) (end 177.046 100.734) (width 1) (layer "F.Cu") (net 1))
 (segment (start 171.326 105.174) (end 172.606 105.174) (width 1) (layer "F.Cu") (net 1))
 (segment (start 187.155 96.774) (end 189.25 96.774) (width 1) (layer "F.Cu") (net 1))
 (segment (start 177.046 100.734) (end 183.195 100.734) (width 1) (layer "F.Cu") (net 1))
 (segment (start 189.23 96.774) (end 185.928 93.472) (width 1) (layer "B.Cu") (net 1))
 (segment (start 189.25 96.774) (end 189.23 96.774) (width 1) (layer "B.Cu") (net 1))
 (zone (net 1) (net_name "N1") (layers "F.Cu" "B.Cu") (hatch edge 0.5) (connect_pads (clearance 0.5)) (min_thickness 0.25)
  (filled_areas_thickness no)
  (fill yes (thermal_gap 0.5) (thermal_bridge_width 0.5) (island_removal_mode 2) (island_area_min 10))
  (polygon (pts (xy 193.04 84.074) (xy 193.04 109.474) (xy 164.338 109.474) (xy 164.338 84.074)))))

